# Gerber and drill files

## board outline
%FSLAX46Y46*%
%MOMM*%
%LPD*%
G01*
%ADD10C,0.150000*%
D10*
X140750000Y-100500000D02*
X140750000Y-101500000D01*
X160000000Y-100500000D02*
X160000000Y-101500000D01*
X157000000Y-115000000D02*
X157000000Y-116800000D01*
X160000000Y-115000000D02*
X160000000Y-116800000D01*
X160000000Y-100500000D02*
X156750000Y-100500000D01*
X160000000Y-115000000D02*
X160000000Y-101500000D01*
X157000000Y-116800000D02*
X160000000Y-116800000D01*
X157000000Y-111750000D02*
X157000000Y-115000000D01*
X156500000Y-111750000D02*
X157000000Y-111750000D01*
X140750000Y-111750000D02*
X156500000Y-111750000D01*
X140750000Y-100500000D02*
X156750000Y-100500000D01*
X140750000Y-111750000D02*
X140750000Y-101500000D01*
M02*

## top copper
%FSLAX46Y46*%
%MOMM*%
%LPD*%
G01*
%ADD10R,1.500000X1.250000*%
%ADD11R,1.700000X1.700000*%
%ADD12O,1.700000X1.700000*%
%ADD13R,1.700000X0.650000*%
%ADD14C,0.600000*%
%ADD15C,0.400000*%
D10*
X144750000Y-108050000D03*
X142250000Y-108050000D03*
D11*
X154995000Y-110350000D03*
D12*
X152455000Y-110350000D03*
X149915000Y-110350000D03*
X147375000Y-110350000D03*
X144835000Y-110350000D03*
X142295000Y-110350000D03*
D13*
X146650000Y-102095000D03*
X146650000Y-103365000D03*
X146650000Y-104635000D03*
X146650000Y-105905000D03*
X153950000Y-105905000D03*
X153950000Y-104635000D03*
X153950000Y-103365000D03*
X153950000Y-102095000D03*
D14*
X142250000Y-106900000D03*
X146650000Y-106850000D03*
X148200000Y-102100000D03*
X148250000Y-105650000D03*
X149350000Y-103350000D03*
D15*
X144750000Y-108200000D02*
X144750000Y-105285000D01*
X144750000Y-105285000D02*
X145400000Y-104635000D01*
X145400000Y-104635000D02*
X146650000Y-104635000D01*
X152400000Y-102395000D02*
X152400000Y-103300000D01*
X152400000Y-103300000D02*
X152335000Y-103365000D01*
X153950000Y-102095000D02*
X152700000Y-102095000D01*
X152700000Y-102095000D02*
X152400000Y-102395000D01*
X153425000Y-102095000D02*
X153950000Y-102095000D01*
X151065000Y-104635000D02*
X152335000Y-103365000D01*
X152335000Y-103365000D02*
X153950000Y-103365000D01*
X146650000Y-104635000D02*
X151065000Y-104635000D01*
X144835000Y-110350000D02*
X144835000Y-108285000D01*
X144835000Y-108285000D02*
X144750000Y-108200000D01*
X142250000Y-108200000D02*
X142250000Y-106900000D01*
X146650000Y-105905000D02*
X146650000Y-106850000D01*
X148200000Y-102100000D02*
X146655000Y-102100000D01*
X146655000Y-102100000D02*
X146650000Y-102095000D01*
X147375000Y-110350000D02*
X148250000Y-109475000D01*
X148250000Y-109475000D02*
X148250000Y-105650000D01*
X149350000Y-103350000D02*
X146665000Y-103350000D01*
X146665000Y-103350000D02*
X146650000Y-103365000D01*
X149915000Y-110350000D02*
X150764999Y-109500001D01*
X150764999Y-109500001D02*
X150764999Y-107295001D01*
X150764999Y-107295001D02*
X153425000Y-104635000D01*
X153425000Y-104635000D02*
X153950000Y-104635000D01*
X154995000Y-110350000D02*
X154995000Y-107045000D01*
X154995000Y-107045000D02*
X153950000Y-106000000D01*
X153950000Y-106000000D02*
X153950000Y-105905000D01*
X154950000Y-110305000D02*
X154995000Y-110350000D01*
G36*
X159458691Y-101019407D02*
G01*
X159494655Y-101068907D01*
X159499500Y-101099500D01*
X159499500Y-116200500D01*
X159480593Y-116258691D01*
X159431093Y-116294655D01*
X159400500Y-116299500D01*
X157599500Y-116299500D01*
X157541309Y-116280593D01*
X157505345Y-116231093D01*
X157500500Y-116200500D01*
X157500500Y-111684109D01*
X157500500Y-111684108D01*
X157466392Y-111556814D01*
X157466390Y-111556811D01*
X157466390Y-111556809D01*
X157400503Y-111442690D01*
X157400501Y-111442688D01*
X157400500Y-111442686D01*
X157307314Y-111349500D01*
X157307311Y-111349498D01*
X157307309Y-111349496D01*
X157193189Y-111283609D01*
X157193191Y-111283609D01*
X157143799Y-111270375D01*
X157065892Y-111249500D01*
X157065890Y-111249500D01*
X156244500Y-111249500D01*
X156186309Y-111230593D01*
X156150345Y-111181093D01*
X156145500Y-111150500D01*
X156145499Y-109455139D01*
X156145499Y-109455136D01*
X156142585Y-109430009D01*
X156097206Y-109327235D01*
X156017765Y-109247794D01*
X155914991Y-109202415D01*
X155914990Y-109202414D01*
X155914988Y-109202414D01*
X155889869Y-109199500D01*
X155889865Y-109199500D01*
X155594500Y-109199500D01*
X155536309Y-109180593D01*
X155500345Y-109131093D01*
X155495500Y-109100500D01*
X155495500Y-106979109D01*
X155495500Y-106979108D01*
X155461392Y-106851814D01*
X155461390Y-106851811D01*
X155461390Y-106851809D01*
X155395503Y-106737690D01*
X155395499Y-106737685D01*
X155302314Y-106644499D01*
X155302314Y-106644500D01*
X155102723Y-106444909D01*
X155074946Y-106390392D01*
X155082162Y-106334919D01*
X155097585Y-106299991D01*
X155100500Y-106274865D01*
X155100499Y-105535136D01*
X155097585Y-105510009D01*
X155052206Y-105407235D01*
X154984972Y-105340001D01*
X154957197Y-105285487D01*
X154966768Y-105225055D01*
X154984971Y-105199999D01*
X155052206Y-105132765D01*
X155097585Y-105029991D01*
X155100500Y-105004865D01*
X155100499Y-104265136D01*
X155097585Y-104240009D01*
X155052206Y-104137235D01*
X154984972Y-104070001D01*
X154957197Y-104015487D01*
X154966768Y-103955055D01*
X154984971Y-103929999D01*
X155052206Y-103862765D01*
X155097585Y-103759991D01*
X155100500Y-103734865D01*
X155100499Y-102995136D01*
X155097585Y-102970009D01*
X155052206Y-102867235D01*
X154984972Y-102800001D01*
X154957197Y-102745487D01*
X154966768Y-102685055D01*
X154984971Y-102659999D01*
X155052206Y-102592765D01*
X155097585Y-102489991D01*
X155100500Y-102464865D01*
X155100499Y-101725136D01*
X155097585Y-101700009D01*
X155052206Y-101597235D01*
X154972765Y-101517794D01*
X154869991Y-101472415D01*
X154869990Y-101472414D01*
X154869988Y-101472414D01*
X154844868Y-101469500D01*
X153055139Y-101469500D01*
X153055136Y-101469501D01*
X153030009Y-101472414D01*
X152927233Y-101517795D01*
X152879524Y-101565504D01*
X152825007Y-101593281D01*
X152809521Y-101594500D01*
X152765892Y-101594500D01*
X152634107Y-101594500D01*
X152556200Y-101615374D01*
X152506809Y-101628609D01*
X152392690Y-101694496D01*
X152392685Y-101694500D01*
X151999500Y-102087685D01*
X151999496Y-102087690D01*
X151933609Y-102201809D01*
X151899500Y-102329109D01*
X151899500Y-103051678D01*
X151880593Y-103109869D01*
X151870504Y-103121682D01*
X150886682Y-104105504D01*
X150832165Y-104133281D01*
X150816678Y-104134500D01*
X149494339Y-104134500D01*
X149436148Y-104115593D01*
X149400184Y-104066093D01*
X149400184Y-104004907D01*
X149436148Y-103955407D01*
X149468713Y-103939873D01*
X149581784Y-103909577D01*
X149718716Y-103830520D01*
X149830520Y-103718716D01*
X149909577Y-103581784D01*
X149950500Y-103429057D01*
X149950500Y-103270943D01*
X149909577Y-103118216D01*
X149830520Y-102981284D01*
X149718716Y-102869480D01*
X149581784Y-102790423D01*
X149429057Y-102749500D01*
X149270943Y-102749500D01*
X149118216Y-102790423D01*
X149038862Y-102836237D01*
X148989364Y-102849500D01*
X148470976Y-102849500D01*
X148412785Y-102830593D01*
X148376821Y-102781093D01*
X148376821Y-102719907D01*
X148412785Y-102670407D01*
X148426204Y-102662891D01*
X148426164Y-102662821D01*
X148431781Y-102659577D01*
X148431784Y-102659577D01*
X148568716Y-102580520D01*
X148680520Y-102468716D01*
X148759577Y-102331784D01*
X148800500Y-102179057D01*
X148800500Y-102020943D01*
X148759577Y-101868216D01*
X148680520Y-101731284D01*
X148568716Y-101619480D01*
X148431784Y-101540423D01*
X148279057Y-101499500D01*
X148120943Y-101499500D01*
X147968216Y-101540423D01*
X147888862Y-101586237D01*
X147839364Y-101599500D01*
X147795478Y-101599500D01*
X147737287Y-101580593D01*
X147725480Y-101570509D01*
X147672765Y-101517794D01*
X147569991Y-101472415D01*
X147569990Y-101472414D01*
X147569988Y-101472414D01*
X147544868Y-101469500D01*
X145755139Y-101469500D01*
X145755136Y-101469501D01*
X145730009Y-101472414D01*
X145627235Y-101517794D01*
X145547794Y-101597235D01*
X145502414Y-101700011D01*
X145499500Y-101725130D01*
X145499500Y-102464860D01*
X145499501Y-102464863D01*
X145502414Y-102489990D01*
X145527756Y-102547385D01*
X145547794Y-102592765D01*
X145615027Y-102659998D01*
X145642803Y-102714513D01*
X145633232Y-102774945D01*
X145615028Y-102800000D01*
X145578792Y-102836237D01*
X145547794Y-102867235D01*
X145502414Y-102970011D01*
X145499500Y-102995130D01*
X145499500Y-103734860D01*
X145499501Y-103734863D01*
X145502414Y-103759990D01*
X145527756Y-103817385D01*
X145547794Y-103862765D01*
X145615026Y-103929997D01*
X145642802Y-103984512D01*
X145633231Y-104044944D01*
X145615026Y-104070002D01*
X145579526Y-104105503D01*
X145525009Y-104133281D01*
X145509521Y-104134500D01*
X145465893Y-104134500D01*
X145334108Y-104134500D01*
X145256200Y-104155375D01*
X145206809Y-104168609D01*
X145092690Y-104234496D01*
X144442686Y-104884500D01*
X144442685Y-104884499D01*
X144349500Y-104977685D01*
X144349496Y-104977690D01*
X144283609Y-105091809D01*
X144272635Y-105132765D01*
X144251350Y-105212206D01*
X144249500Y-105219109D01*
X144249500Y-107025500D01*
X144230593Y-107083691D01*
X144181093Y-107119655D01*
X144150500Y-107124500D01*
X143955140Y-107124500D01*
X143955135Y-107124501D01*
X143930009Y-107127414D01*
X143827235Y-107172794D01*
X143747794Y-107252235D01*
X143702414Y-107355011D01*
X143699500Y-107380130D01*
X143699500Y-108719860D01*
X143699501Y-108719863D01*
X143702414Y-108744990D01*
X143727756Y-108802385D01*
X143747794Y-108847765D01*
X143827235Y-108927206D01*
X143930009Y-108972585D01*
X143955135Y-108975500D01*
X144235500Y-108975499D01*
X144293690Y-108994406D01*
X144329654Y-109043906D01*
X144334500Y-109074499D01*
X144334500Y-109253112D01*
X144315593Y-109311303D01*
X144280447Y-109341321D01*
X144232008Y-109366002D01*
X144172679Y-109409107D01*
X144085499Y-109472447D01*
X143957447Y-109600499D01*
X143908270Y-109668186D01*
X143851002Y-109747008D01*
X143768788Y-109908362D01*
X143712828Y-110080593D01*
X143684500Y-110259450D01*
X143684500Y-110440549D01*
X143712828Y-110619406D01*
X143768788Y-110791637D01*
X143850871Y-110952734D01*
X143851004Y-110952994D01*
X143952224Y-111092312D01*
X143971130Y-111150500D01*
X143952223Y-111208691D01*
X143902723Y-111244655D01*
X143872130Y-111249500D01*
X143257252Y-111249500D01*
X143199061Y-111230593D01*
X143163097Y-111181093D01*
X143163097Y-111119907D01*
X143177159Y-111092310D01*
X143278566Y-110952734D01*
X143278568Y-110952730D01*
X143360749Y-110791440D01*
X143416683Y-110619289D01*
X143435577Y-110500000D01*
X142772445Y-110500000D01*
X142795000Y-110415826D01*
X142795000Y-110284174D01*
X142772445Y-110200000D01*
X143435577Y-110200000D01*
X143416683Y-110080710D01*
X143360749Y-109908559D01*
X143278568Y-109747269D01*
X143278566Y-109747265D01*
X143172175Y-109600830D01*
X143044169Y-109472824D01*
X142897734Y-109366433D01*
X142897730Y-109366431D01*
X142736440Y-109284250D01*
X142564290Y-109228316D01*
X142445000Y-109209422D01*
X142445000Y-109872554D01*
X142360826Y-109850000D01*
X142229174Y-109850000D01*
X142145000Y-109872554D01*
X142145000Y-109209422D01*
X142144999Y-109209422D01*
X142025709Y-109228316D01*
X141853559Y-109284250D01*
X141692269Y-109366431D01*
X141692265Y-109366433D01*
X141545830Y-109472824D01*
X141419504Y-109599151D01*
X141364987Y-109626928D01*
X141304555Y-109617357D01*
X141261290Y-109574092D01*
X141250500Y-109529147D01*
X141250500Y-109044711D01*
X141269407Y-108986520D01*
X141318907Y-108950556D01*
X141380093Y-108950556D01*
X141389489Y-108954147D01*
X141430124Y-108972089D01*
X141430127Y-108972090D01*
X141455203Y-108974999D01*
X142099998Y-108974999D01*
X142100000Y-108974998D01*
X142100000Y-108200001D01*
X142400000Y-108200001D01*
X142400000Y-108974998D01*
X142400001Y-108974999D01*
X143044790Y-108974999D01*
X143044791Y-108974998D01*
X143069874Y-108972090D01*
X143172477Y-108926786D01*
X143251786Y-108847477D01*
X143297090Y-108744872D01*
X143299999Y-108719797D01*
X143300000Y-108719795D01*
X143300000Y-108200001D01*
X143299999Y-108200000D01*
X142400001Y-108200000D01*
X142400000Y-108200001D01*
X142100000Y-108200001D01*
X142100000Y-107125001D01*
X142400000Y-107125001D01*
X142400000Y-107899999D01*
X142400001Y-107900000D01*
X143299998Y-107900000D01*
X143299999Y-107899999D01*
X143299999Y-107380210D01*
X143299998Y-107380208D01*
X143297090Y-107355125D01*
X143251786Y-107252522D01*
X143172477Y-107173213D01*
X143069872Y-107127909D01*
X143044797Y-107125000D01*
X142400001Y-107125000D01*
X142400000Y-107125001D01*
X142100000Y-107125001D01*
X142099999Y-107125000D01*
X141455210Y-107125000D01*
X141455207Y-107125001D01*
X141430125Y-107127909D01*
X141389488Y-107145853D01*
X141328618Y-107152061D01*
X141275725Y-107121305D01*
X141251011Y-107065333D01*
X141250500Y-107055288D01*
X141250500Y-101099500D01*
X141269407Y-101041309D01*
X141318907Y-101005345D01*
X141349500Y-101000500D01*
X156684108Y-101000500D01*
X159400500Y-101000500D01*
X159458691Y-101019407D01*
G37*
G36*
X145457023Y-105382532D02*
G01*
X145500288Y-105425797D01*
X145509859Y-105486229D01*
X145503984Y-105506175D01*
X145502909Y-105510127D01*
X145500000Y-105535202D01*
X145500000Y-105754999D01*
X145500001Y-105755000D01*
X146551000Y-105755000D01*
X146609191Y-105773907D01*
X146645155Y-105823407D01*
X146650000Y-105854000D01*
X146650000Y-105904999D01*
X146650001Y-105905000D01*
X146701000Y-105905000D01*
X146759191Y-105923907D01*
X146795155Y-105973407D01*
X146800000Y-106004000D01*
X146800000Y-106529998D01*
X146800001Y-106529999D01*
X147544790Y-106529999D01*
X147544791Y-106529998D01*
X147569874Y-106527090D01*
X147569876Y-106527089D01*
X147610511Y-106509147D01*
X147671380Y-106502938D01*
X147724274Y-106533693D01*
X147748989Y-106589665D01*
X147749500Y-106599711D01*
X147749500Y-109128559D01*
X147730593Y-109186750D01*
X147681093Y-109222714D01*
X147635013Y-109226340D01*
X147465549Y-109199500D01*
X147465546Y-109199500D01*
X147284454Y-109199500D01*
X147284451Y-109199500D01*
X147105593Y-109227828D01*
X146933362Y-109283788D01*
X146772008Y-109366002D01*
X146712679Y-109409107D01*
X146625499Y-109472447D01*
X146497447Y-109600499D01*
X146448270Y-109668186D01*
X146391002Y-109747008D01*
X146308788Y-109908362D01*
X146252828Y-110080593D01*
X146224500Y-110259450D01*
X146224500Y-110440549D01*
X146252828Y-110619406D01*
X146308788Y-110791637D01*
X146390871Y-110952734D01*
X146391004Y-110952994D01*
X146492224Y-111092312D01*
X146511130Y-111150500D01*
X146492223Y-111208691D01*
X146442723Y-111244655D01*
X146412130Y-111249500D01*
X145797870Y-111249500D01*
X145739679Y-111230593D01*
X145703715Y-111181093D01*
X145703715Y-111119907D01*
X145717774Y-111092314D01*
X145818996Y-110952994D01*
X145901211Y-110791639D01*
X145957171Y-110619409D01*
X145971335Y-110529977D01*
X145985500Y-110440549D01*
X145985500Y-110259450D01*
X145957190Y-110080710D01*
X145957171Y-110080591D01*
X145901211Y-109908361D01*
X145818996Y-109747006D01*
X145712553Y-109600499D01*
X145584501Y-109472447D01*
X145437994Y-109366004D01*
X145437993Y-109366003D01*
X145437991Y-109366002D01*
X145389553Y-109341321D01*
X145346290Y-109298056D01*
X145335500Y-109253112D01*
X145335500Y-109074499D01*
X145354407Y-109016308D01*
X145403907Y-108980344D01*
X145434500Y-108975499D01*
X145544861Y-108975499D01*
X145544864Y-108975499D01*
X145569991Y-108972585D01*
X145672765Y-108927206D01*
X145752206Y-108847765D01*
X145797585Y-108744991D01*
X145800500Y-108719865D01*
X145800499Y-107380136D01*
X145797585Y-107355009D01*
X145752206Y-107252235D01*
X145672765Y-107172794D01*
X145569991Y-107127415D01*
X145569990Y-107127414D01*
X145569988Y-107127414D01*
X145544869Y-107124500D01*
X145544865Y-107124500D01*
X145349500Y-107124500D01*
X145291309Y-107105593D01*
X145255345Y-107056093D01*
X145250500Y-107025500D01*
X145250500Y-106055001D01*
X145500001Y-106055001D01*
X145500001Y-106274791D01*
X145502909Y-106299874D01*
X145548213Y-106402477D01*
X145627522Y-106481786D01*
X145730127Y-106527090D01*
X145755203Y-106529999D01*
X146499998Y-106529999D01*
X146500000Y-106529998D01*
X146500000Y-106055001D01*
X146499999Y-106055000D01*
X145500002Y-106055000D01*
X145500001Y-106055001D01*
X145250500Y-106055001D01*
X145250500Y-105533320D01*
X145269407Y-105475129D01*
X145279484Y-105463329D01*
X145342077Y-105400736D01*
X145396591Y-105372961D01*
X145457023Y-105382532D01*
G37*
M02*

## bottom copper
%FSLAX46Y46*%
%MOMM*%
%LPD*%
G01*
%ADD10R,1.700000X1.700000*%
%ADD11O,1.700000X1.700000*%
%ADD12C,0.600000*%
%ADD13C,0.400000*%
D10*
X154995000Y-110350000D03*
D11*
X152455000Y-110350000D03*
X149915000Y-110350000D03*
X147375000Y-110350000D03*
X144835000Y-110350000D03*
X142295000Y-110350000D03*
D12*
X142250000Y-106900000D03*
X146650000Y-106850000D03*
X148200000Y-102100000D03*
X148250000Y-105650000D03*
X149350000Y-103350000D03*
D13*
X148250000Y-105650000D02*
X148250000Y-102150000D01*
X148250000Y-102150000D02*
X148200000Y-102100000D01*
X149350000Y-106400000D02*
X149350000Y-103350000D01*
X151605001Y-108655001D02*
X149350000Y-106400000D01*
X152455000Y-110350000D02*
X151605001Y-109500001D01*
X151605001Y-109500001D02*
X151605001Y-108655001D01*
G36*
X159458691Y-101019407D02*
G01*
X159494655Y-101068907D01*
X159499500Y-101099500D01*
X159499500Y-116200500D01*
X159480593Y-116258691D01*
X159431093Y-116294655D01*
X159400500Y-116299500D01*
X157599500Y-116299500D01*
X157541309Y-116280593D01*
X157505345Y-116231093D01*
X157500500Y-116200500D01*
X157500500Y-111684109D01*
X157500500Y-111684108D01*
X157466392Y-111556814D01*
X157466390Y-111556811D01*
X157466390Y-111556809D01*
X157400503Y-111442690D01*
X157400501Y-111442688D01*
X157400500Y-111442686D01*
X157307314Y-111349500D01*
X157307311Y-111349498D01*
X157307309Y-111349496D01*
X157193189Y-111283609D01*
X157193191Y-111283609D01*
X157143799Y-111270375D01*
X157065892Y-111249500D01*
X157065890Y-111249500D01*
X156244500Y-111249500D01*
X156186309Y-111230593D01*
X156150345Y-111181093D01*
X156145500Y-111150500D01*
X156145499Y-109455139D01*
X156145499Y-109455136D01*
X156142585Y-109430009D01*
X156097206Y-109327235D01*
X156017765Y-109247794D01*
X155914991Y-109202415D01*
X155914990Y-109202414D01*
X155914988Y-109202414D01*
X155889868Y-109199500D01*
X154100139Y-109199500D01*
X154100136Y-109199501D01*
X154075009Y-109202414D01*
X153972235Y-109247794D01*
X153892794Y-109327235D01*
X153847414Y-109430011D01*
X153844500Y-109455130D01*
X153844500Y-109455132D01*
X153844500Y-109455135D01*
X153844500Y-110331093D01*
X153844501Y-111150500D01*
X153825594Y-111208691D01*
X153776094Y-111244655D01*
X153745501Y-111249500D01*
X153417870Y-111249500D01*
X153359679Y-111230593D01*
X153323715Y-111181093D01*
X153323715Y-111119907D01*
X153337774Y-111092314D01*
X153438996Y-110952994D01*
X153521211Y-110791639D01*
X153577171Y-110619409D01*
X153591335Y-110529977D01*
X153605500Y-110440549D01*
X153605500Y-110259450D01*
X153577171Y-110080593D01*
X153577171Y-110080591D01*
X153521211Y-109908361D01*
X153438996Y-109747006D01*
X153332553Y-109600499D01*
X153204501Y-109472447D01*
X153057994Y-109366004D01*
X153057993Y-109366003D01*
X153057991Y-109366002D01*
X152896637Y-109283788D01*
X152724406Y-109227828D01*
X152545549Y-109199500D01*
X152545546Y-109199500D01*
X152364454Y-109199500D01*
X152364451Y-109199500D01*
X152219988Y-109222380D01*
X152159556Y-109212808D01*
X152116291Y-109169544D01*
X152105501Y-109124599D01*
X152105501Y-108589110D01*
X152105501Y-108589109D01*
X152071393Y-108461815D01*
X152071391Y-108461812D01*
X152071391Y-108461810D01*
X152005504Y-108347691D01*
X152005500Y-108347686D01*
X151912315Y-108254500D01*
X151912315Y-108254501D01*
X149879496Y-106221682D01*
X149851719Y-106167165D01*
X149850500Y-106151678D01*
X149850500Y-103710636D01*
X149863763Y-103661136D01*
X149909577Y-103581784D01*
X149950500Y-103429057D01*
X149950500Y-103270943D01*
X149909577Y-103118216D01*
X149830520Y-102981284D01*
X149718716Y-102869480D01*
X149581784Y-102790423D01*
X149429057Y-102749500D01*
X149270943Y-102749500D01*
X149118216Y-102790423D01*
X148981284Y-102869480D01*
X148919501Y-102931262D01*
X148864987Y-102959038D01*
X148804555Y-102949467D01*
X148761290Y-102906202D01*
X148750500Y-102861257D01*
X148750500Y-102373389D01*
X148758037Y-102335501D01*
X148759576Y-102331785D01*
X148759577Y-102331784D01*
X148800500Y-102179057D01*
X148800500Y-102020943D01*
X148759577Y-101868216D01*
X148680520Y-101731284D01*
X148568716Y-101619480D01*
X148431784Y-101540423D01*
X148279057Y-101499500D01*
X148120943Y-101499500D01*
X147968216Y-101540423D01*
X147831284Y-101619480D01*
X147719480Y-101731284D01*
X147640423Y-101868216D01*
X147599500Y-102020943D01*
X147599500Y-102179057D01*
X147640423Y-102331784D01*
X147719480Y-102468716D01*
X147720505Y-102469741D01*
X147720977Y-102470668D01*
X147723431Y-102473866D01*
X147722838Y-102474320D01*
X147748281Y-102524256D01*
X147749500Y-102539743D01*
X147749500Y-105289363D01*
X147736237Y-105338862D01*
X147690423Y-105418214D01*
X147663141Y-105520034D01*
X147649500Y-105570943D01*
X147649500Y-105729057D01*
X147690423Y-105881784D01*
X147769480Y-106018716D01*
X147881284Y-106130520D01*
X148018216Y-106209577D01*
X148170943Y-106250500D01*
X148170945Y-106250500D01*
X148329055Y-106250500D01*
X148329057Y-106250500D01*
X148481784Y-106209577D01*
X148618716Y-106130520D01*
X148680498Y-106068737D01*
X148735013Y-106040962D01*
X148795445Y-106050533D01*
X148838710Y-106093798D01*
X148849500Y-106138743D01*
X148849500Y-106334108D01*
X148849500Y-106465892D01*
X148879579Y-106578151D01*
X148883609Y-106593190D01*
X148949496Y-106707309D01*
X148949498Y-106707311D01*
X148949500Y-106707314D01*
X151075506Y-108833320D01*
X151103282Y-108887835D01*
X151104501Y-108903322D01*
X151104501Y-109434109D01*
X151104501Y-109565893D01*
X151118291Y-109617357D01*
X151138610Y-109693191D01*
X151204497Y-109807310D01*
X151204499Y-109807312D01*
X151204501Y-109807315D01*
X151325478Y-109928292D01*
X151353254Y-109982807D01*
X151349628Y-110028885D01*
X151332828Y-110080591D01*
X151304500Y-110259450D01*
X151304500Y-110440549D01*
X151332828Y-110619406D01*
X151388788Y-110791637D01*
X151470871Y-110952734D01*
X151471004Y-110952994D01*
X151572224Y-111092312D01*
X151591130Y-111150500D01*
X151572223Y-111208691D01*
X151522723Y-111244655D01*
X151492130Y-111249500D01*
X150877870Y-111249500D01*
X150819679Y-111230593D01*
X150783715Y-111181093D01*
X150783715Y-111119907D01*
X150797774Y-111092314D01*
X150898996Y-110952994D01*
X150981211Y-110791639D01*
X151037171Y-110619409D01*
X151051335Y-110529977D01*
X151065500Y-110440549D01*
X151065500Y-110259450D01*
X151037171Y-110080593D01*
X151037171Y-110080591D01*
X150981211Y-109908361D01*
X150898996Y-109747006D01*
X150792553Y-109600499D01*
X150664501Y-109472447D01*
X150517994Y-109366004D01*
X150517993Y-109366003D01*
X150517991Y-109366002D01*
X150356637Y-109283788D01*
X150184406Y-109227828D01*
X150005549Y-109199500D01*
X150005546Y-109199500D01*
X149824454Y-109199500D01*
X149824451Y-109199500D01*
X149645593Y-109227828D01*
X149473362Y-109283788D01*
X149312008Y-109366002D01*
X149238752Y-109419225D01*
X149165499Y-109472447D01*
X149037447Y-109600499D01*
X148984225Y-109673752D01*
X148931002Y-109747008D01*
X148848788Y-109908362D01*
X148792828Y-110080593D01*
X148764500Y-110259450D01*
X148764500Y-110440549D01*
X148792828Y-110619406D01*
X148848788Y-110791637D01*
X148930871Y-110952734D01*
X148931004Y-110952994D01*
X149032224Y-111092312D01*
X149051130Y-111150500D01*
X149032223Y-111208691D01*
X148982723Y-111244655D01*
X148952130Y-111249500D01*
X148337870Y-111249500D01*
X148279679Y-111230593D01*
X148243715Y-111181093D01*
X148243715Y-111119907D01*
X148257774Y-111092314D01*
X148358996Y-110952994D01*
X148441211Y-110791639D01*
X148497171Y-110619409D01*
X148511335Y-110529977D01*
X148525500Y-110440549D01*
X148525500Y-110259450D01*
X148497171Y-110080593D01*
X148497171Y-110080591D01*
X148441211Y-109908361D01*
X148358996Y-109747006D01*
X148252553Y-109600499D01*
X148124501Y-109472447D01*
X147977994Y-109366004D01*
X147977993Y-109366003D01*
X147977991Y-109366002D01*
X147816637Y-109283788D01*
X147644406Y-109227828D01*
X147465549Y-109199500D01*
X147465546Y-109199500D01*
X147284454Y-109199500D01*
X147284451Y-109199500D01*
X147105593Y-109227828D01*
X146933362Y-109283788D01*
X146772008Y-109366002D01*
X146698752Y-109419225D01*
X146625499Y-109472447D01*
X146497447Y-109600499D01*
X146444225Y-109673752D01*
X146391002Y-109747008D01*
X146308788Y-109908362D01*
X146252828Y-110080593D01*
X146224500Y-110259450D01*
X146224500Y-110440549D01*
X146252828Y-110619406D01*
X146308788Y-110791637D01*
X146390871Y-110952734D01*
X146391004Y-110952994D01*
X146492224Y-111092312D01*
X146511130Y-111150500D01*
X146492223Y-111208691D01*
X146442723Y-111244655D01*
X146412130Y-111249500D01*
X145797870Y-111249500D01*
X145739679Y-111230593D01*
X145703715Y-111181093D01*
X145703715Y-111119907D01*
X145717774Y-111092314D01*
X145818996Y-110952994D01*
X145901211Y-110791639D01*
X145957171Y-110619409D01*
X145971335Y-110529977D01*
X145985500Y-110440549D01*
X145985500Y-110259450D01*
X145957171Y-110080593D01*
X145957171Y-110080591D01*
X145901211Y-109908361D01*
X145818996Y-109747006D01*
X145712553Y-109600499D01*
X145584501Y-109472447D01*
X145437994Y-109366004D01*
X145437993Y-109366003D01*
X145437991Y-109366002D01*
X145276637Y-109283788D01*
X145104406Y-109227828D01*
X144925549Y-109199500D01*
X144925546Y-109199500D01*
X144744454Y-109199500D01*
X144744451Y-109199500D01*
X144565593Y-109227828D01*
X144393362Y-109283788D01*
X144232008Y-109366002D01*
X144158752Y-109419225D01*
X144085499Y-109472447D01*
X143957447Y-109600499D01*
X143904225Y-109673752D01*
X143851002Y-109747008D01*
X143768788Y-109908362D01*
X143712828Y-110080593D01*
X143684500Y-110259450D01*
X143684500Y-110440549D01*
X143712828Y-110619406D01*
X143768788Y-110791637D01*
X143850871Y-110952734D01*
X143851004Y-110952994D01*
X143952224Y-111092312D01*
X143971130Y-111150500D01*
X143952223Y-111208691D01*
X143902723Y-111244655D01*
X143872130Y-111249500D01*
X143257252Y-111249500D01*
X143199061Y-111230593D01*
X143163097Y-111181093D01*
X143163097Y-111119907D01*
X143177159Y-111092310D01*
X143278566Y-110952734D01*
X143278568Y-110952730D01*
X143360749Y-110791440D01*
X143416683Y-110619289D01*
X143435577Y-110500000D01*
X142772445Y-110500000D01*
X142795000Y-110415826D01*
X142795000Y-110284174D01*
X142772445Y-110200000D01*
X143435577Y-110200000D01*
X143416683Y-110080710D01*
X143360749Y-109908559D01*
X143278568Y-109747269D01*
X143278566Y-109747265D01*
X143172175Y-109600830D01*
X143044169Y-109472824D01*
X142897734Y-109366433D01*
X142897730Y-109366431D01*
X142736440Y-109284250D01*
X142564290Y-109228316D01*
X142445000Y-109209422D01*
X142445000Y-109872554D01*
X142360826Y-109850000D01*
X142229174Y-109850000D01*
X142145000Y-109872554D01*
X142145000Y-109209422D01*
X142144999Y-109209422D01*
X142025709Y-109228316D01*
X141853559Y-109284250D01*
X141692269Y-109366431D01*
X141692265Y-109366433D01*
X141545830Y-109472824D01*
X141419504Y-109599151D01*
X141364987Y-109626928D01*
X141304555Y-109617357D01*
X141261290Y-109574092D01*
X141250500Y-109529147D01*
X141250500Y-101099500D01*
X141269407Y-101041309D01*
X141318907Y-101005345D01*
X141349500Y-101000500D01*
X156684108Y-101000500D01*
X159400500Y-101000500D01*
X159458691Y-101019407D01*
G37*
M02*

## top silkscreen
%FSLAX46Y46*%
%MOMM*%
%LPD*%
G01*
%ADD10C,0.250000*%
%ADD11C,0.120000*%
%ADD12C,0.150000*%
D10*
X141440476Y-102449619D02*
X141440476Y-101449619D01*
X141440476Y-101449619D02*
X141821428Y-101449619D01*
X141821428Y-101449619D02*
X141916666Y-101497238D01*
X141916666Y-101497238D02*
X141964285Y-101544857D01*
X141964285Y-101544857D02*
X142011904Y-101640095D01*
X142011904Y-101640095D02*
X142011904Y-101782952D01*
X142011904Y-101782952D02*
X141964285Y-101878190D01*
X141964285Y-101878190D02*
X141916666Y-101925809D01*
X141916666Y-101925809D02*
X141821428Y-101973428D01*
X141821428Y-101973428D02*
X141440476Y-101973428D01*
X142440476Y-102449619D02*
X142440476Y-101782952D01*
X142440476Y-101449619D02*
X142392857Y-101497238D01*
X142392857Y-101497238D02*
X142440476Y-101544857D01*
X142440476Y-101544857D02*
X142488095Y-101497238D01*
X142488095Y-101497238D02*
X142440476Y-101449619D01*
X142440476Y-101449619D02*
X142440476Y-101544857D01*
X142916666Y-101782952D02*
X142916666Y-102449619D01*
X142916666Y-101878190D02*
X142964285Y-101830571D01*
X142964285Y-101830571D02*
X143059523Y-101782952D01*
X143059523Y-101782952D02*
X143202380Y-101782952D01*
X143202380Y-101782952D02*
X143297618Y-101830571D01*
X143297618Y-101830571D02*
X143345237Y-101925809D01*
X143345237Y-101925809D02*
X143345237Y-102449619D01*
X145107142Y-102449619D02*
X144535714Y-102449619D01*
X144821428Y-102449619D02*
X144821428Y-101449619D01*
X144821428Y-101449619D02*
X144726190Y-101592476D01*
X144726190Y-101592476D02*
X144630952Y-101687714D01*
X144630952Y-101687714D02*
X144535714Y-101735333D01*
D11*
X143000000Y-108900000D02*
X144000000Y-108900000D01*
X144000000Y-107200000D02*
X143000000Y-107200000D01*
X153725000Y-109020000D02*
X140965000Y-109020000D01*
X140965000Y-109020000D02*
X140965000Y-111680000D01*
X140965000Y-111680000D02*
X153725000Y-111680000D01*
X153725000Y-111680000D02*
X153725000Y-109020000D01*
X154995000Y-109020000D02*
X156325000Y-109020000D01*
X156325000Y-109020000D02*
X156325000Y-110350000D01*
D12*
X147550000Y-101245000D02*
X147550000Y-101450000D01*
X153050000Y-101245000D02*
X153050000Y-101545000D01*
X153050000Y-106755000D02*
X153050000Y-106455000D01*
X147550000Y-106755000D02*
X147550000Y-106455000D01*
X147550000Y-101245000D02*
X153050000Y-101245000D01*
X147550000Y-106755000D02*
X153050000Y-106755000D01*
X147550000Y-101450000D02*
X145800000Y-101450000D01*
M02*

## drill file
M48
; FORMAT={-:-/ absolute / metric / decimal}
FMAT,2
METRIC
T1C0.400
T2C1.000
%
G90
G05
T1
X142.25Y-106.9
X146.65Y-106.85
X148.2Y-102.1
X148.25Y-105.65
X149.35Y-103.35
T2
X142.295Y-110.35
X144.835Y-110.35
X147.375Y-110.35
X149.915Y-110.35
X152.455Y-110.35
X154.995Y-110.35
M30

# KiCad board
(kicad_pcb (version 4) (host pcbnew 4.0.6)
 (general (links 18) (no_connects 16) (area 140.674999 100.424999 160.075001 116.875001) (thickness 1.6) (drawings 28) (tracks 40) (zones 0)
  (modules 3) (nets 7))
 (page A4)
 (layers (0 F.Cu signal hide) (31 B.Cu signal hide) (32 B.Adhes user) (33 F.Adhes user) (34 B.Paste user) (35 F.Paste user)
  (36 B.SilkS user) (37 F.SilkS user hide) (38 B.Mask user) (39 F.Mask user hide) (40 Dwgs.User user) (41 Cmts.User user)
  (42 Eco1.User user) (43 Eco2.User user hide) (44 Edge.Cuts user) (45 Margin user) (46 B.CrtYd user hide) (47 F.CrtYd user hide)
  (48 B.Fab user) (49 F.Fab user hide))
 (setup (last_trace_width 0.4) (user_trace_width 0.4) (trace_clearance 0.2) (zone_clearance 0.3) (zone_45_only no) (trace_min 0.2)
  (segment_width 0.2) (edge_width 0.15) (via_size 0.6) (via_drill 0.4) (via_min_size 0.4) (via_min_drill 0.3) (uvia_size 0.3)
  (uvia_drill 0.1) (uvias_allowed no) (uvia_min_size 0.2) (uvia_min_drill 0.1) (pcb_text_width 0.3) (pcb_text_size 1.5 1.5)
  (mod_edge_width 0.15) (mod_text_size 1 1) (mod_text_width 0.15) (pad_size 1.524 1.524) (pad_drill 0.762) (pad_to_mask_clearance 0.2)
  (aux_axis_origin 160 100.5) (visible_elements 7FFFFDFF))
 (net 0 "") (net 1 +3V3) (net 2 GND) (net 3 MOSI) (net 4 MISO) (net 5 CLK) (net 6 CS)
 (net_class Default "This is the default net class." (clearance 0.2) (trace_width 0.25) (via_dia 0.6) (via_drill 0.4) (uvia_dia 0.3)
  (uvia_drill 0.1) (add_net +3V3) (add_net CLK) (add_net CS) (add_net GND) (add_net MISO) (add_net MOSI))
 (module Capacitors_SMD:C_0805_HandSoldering (layer F.Cu) (at 143.5 108.05 180)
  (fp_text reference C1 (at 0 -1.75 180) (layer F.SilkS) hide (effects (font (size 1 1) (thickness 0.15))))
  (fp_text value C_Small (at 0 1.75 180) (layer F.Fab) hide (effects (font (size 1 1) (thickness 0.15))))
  (fp_line (start 0.5 -0.85) (end -0.5 -0.85) (layer F.SilkS) (width 0.12))
  (fp_line (start -0.5 0.85) (end 0.5 0.85) (layer F.SilkS) (width 0.12))
  (pad 1 smd rect (at -1.25 0 180) (size 1.5 1.25) (layers F.Cu F.Paste F.Mask) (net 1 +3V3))
  (pad 2 smd rect (at 1.25 0 180) (size 1.5 1.25) (layers F.Cu F.Paste F.Mask) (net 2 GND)))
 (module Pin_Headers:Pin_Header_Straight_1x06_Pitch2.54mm (layer F.Cu) (at 154.995 110.35 270)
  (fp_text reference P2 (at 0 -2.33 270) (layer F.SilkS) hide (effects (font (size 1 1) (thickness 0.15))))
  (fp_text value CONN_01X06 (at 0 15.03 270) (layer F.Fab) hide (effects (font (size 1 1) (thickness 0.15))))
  (fp_line (start -1.33 1.27) (end -1.33 14.03) (layer F.SilkS) (width 0.12))
  (fp_line (start -1.33 14.03) (end 1.33 14.03) (layer F.SilkS) (width 0.12))
  (fp_line (start 1.33 14.03) (end 1.33 1.27) (layer F.SilkS) (width 0.12))
  (fp_line (start 1.33 1.27) (end -1.33 1.27) (layer F.SilkS) (width 0.12))
  (fp_line (start -1.33 0) (end -1.33 -1.33) (layer F.SilkS) (width 0.12))
  (fp_line (start -1.33 -1.33) (end 0 -1.33) (layer F.SilkS) (width 0.12))
  (pad 1 thru_hole rect (at 0 0 270) (size 1.7 1.7) (drill 1) (layers *.Cu *.Mask) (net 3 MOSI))
  (pad 2 thru_hole oval (at 0 2.54 270) (size 1.7 1.7) (drill 1) (layers *.Cu *.Mask) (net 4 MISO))
  (pad 3 thru_hole oval (at 0 5.08 270) (size 1.7 1.7) (drill 1) (layers *.Cu *.Mask) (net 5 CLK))
  (pad 4 thru_hole oval (at 0 7.62 270) (size 1.7 1.7) (drill 1) (layers *.Cu *.Mask) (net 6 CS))
  (pad 5 thru_hole oval (at 0 10.16 270) (size 1.7 1.7) (drill 1) (layers *.Cu *.Mask) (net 1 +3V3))
  (pad 6 thru_hole oval (at 0 12.7 270) (size 1.7 1.7) (drill 1) (layers *.Cu *.Mask) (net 2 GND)))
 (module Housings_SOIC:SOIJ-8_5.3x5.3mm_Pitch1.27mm (layer F.Cu) (at 150.3 104)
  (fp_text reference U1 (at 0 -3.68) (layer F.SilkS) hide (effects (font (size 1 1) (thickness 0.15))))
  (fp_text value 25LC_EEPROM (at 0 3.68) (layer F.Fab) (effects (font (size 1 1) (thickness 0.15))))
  (fp_line (start -2.75 -2.755) (end -2.75 -2.55) (layer F.SilkS) (width 0.15))
  (fp_line (start 2.75 -2.755) (end 2.75 -2.455) (layer F.SilkS) (width 0.15))
  (fp_line (start 2.75 2.755) (end 2.75 2.455) (layer F.SilkS) (width 0.15))
  (fp_line (start -2.75 2.755) (end -2.75 2.455) (layer F.SilkS) (width 0.15))
  (fp_line (start -2.75 -2.755) (end 2.75 -2.755) (layer F.SilkS) (width 0.15))
  (fp_line (start -2.75 2.755) (end 2.75 2.755) (layer F.SilkS) (width 0.15))
  (fp_line (start -2.75 -2.55) (end -4.5 -2.55) (layer F.SilkS) (width 0.15))
  (pad 1 smd rect (at -3.65 -1.905) (size 1.7 0.65) (layers F.Cu F.Paste F.Mask) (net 6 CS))
  (pad 2 smd rect (at -3.65 -0.635) (size 1.7 0.65) (layers F.Cu F.Paste F.Mask) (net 4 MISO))
  (pad 3 smd rect (at -3.65 0.635) (size 1.7 0.65) (layers F.Cu F.Paste F.Mask) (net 1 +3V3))
  (pad 4 smd rect (at -3.65 1.905) (size 1.7 0.65) (layers F.Cu F.Paste F.Mask) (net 2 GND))
  (pad 5 smd rect (at 3.65 1.905) (size 1.7 0.65) (layers F.Cu F.Paste F.Mask) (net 3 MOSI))
  (pad 6 smd rect (at 3.65 0.635) (size 1.7 0.65) (layers F.Cu F.Paste F.Mask) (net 5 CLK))
  (pad 7 smd rect (at 3.65 -0.635) (size 1.7 0.65) (layers F.Cu F.Paste F.Mask) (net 1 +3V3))
  (pad 8 smd rect (at 3.65 -1.905) (size 1.7 0.65) (layers F.Cu F.Paste F.Mask) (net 1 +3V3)))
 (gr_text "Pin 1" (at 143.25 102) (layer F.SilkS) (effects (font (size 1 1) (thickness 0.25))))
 (gr_line (start 140.75 100.5) (end 140.75 101.5) (layer Edge.Cuts) (width 0.15))
 (gr_line (start 160 100.5) (end 160 101.5) (layer Edge.Cuts) (width 0.15))
 (gr_line (start 157 115) (end 157 116.8) (layer Edge.Cuts) (width 0.15))
 (gr_line (start 160 115) (end 160 116.8) (layer Edge.Cuts) (width 0.15))
 (gr_line (start 160 100.5) (end 156.75 100.5) (layer Edge.Cuts) (width 0.15))
 (gr_line (start 160 115) (end 160 101.5) (layer Edge.Cuts) (width 0.15))
 (gr_line (start 157 116.8) (end 160 116.8) (layer Edge.Cuts) (width 0.15))
 (gr_line (start 157 111.75) (end 157 115) (layer Edge.Cuts) (width 0.15))
 (gr_line (start 156.5 111.75) (end 157 111.75) (layer Edge.Cuts) (width 0.15))
 (gr_line (start 140.75 111.75) (end 156.5 111.75) (layer Edge.Cuts) (width 0.15))
 (gr_line (start 140.75 100.5) (end 156.75 100.5) (layer Edge.Cuts) (width 0.15))
 (gr_line (start 140.75 111.75) (end 140.75 101.5) (layer Edge.Cuts) (width 0.15))
 (segment (start 144.75 108.2) (end 144.75 105.285) (width 0.4) (layer F.Cu) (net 1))
 (segment (start 144.75 105.285) (end 145.4 104.635) (width 0.4) (layer F.Cu) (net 1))
 (segment (start 145.4 104.635) (end 146.65 104.635) (width 0.4) (layer F.Cu) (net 1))
 (segment (start 152.4 102.395) (end 152.4 103.3) (width 0.4) (layer F.Cu) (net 1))
 (segment (start 152.4 103.3) (end 152.335 103.365) (width 0.4) (layer F.Cu) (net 1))
 (segment (start 153.95 102.095) (end 152.7 102.095) (width 0.4) (layer F.Cu) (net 1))
 (segment (start 152.7 102.095) (end 152.4 102.395) (width 0.4) (layer F.Cu) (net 1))
 (segment (start 153.425 102.095) (end 153.95 102.095) (width 0.4) (layer F.Cu) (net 1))
 (segment (start 151.065 104.635) (end 152.335 103.365) (width 0.4) (layer F.Cu) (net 1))
 (segment (start 152.335 103.365) (end 153.95 103.365) (width 0.4) (layer F.Cu) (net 1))
 (segment (start 146.65 104.635) (end 151.065 104.635) (width 0.4) (layer F.Cu) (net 1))
 (segment (start 144.835 110.35) (end 144.835 108.285) (width 0.4) (layer F.Cu) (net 1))
 (segment (start 144.835 108.285) (end 144.75 108.2) (width 0.4) (layer F.Cu) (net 1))
 (segment (start 142.25 108.2) (end 142.25 106.9) (width 0.4) (layer F.Cu) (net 2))
 (via (at 142.25 106.9) (size 0.6) (drill 0.4) (layers F.Cu B.Cu) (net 2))
 (segment (start 146.65 105.905) (end 146.65 106.85) (width 0.4) (layer F.Cu) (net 2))
 (via (at 146.65 106.85) (size 0.6) (drill 0.4) (layers F.Cu B.Cu) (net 2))
 (segment (start 148.2 102.1) (end 146.655 102.1) (width 0.4) (layer F.Cu) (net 6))
 (segment (start 146.655 102.1) (end 146.65 102.095) (width 0.4) (layer F.Cu) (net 6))
 (segment (start 148.25 105.65) (end 148.25 102.15) (width 0.4) (layer B.Cu) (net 6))
 (segment (start 148.25 102.15) (end 148.2 102.1) (width 0.4) (layer B.Cu) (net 6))
 (via (at 148.2 102.1) (size 0.6) (drill 0.4) (layers F.Cu B.Cu) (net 6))
 (segment (start 147.375 110.35) (end 148.25 109.475) (width 0.4) (layer F.Cu) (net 6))
 (segment (start 148.25 109.475) (end 148.25 105.65) (width 0.4) (layer F.Cu) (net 6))
 (via (at 148.25 105.65) (size 0.6) (drill 0.4) (layers F.Cu B.Cu) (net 6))
 (segment (start 149.35 103.35) (end 146.665 103.35) (width 0.4) (layer F.Cu) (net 4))
 (segment (start 146.665 103.35) (end 146.65 103.365) (width 0.4) (layer F.Cu) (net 4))
 (segment (start 149.35 106.4) (end 149.35 103.35) (width 0.4) (layer B.Cu) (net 4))
 (via (at 149.35 103.35) (size 0.6) (drill 0.4) (layers F.Cu B.Cu) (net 4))
 (segment (start 151.605001 108.655001) (end 149.35 106.4) (width 0.4) (layer B.Cu) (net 4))
 (segment (start 152.455 110.35) (end 151.605001 109.500001) (width 0.4) (layer B.Cu) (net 4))
 (segment (start 151.605001 109.500001) (end 151.605001 108.655001) (width 0.4) (layer B.Cu) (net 4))
 (segment (start 149.915 110.35) (end 150.764999 109.500001) (width 0.4) (layer F.Cu) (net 5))
 (segment (start 150.764999 109.500001) (end 150.764999 107.295001) (width 0.4) (layer F.Cu) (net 5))
 (segment (start 150.764999 107.295001) (end 153.425 104.635) (width 0.4) (layer F.Cu) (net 5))
 (segment (start 153.425 104.635) (end 153.95 104.635) (width 0.4) (layer F.Cu) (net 5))
 (segment (start 154.995 110.35) (end 154.995 107.045) (width 0.4) (layer F.Cu) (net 3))
 (segment (start 154.995 107.045) (end 153.95 106) (width 0.4) (layer F.Cu) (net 3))
 (segment (start 153.95 106) (end 153.95 105.905) (width 0.4) (layer F.Cu) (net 3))
 (segment (start 154.95 110.305) (end 154.995 110.35) (width 0.4) (layer F.Cu) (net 3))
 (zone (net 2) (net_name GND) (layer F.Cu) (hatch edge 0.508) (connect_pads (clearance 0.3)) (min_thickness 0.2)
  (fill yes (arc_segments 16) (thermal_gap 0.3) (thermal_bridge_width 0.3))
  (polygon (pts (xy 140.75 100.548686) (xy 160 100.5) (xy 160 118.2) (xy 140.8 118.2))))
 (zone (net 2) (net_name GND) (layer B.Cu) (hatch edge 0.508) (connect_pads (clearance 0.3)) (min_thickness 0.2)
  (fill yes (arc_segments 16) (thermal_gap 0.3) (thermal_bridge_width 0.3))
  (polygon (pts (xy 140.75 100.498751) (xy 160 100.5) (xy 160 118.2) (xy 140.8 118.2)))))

